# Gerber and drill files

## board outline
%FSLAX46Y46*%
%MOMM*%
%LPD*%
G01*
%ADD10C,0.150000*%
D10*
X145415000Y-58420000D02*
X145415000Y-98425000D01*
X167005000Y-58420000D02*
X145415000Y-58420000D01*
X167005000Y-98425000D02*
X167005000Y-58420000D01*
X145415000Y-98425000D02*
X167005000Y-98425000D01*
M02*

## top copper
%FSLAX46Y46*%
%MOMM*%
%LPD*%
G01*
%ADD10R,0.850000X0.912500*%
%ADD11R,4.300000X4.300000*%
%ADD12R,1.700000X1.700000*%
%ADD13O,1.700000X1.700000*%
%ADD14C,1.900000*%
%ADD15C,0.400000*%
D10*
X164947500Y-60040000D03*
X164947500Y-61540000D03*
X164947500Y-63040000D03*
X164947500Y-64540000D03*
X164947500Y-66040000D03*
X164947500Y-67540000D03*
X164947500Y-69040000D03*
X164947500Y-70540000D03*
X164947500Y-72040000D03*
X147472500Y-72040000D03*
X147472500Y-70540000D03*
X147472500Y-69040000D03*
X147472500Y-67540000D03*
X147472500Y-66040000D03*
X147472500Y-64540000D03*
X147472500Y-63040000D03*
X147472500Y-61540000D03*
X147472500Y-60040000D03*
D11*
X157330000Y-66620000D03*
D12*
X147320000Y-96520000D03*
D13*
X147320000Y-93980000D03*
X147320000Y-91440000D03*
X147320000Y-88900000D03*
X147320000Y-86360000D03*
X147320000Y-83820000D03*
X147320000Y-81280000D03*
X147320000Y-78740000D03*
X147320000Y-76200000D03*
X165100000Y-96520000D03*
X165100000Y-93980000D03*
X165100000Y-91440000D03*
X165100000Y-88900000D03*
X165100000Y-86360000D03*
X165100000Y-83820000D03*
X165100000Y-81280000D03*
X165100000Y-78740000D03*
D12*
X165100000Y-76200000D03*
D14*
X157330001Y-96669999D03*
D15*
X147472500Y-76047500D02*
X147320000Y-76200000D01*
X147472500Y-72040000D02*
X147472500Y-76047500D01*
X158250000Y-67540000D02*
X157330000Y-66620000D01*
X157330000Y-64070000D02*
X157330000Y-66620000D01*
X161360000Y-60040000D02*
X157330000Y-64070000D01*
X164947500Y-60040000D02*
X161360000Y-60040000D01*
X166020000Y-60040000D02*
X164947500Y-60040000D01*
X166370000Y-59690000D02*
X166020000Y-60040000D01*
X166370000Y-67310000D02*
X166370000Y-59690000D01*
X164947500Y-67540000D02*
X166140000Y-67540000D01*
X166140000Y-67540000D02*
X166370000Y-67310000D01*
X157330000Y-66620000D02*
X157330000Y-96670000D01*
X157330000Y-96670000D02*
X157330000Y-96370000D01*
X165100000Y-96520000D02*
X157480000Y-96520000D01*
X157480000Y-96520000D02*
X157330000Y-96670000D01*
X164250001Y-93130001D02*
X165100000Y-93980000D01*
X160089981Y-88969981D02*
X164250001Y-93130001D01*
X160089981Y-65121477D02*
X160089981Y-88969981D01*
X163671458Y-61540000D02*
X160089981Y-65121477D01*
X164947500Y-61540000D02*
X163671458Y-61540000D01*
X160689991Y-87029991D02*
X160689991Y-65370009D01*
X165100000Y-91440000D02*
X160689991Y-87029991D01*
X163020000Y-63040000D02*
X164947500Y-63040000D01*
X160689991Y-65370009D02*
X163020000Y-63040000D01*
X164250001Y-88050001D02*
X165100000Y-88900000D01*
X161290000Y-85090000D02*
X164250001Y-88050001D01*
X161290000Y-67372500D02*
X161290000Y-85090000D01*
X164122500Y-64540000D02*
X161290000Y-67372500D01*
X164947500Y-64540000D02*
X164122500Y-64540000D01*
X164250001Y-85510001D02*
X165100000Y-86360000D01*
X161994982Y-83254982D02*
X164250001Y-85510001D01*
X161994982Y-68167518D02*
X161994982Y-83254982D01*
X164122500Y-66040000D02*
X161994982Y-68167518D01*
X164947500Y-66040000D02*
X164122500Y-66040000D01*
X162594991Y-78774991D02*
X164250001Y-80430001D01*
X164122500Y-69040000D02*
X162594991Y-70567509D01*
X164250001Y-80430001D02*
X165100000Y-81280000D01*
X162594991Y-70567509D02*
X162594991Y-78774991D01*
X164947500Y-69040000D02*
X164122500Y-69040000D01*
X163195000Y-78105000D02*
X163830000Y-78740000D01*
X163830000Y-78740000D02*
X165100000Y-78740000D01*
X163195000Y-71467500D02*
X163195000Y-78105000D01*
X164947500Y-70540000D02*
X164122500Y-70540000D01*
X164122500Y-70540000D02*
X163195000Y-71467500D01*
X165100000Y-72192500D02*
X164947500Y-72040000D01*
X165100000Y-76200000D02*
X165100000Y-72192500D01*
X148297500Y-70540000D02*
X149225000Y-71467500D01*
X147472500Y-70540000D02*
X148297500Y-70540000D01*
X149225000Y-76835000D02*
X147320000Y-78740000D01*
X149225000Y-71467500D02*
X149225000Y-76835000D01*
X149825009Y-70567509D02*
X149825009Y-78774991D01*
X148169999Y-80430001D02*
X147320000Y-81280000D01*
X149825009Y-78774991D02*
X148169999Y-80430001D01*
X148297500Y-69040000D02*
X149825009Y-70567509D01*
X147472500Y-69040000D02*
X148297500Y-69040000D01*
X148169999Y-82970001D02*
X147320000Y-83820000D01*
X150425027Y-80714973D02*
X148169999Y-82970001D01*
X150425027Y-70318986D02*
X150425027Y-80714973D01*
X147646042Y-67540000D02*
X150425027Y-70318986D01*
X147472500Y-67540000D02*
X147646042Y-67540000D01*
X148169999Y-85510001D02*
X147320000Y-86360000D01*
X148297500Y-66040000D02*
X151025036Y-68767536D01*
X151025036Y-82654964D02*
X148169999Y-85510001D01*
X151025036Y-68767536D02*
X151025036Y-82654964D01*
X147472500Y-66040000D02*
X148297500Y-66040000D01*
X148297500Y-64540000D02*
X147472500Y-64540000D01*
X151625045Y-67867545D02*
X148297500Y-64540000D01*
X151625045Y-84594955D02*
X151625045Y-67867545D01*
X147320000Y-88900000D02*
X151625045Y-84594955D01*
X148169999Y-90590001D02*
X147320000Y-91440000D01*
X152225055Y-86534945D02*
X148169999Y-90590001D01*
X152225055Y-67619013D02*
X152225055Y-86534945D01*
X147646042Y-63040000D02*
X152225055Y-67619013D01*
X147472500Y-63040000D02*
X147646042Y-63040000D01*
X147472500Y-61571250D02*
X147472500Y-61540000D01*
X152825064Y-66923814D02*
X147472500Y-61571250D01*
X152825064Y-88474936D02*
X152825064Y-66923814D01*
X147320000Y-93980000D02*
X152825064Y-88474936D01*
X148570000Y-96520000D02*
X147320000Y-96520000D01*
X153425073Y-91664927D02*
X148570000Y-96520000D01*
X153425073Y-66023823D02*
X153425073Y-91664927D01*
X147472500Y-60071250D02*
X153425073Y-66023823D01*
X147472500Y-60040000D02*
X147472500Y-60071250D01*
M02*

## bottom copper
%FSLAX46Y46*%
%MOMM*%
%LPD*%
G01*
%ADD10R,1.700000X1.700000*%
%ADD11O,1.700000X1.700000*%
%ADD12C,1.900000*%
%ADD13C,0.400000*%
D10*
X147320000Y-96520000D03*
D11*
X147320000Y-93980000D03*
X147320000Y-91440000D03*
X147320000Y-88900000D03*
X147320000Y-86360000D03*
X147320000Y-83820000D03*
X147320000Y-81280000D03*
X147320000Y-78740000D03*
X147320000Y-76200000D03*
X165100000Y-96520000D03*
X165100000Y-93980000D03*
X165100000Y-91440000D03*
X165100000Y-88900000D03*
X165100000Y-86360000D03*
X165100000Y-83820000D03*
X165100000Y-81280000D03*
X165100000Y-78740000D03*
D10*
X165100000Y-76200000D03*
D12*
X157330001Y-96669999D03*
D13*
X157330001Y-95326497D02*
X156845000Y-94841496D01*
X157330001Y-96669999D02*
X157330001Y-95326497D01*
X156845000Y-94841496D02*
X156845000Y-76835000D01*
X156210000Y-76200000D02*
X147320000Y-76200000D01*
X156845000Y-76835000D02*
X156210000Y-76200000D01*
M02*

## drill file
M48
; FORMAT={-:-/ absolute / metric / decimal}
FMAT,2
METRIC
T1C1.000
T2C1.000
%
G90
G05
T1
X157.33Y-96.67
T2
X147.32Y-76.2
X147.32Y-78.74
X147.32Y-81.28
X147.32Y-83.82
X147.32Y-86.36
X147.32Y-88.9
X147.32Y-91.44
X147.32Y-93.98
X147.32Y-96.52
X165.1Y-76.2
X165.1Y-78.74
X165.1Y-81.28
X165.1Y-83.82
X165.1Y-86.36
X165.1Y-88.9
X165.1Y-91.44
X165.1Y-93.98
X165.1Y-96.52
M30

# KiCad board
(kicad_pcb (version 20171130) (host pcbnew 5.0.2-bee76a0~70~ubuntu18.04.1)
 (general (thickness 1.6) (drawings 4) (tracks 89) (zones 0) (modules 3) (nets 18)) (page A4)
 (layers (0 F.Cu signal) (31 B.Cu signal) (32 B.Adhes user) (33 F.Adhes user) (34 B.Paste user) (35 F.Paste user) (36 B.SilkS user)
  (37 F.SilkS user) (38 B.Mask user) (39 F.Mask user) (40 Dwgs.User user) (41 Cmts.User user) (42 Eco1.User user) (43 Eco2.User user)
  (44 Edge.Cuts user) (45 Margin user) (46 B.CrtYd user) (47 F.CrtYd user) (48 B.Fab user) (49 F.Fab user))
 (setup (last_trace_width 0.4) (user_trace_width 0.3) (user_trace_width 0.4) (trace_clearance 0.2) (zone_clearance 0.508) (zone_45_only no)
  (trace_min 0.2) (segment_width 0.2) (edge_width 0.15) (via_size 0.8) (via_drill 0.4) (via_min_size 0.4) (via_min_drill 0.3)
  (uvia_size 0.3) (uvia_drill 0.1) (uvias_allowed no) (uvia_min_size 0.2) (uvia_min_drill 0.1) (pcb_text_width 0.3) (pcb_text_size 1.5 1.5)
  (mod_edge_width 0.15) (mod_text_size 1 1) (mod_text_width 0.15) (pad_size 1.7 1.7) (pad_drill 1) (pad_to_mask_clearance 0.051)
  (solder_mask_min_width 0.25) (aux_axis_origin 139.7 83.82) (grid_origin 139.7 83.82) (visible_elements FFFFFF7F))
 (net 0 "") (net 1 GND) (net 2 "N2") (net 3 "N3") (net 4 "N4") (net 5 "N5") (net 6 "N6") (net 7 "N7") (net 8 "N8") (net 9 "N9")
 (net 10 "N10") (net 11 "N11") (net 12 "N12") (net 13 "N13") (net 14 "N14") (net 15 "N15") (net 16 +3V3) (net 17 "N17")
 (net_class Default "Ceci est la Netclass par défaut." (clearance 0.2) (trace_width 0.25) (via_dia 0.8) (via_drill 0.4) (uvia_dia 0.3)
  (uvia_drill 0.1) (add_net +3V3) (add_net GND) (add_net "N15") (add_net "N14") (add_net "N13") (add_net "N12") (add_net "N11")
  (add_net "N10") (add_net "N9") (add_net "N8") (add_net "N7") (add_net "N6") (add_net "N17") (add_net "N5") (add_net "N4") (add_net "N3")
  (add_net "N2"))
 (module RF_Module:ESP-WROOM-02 (layer F.Cu) (at 156.21 66.04)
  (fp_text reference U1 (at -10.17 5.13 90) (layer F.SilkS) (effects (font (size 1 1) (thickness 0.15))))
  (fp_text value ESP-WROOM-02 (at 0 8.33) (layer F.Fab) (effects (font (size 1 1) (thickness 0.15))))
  (pad 18 smd rect (at 8.7375 -6) (size 0.85 0.9125) (layers F.Cu F.Paste F.Mask) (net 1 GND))
  (pad 17 smd rect (at 8.7375 -4.5) (size 0.85 0.9125) (layers F.Cu F.Paste F.Mask) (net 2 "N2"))
  (pad 16 smd rect (at 8.7375 -3) (size 0.85 0.9125) (layers F.Cu F.Paste F.Mask) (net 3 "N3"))
  (pad 15 smd rect (at 8.7375 -1.5) (size 0.85 0.9125) (layers F.Cu F.Paste F.Mask) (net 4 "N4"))
  (pad 14 smd rect (at 8.7375 0) (size 0.85 0.9125) (layers F.Cu F.Paste F.Mask) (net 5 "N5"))
  (pad 13 smd rect (at 8.7375 1.5) (size 0.85 0.9125) (layers F.Cu F.Paste F.Mask) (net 1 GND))
  (pad 12 smd rect (at 8.7375 3) (size 0.85 0.9125) (layers F.Cu F.Paste F.Mask) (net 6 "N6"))
  (pad 11 smd rect (at 8.7375 4.5) (size 0.85 0.9125) (layers F.Cu F.Paste F.Mask) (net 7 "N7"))
  (pad 10 smd rect (at 8.7375 6) (size 0.85 0.9125) (layers F.Cu F.Paste F.Mask) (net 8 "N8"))
  (pad 9 smd rect (at -8.7375 6) (size 0.85 0.9125) (layers F.Cu F.Paste F.Mask) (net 1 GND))
  (pad 8 smd rect (at -8.7375 4.5) (size 0.85 0.9125) (layers F.Cu F.Paste F.Mask) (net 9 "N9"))
  (pad 7 smd rect (at -8.7375 3) (size 0.85 0.9125) (layers F.Cu F.Paste F.Mask) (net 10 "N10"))
  (pad 6 smd rect (at -8.7375 1.5) (size 0.85 0.9125) (layers F.Cu F.Paste F.Mask) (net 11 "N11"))
  (pad 5 smd rect (at -8.7375 0) (size 0.85 0.9125) (layers F.Cu F.Paste F.Mask) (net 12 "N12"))
  (pad 4 smd rect (at -8.7375 -1.5) (size 0.85 0.9125) (layers F.Cu F.Paste F.Mask) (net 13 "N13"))
  (pad 3 smd rect (at -8.7375 -3) (size 0.85 0.9125) (layers F.Cu F.Paste F.Mask) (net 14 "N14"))
  (pad 2 smd rect (at -8.7375 -4.5) (size 0.85 0.9125) (layers F.Cu F.Paste F.Mask) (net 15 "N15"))
  (pad 1 smd rect (at -8.7375 -6) (size 0.85 0.9125) (layers F.Cu F.Paste F.Mask) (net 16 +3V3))
  (pad 19 smd rect (at 1.12 0.58) (size 4.3 4.3) (layers F.Cu F.Paste F.Mask) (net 1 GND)))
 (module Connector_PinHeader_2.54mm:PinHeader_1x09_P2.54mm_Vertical (layer F.Cu) (at 147.32 96.52 180)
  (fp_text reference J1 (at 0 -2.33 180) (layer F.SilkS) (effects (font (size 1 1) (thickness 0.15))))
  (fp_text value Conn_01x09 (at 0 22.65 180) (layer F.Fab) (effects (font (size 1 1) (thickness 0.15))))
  (pad 1 thru_hole rect (at 0 0 180) (size 1.7 1.7) (drill 1) (layers *.Cu *.Mask) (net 16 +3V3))
  (pad 2 thru_hole oval (at 0 2.54 180) (size 1.7 1.7) (drill 1) (layers *.Cu *.Mask) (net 15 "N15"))
  (pad 3 thru_hole oval (at 0 5.08 180) (size 1.7 1.7) (drill 1) (layers *.Cu *.Mask) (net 14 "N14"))
  (pad 4 thru_hole oval (at 0 7.62 180) (size 1.7 1.7) (drill 1) (layers *.Cu *.Mask) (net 13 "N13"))
  (pad 5 thru_hole oval (at 0 10.16 180) (size 1.7 1.7) (drill 1) (layers *.Cu *.Mask) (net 12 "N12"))
  (pad 6 thru_hole oval (at 0 12.7 180) (size 1.7 1.7) (drill 1) (layers *.Cu *.Mask) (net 11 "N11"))
  (pad 7 thru_hole oval (at 0 15.24 180) (size 1.7 1.7) (drill 1) (layers *.Cu *.Mask) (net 10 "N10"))
  (pad 8 thru_hole oval (at 0 17.78 180) (size 1.7 1.7) (drill 1) (layers *.Cu *.Mask) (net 9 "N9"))
  (pad 9 thru_hole oval (at 0 20.32 180) (size 1.7 1.7) (drill 1) (layers *.Cu *.Mask) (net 1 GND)))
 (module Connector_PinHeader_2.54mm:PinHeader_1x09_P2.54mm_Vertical (layer F.Cu) (at 165.1 76.2)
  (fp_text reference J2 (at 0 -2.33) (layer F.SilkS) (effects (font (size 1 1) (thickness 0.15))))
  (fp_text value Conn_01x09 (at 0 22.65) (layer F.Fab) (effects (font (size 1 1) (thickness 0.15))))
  (pad 9 thru_hole oval (at 0 20.32) (size 1.7 1.7) (drill 1) (layers *.Cu *.Mask) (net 1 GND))
  (pad 8 thru_hole oval (at 0 17.78) (size 1.7 1.7) (drill 1) (layers *.Cu *.Mask) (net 2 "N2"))
  (pad 7 thru_hole oval (at 0 15.24) (size 1.7 1.7) (drill 1) (layers *.Cu *.Mask) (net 3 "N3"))
  (pad 6 thru_hole oval (at 0 12.7) (size 1.7 1.7) (drill 1) (layers *.Cu *.Mask) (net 4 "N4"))
  (pad 5 thru_hole oval (at 0 10.16) (size 1.7 1.7) (drill 1) (layers *.Cu *.Mask) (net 5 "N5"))
  (pad 4 thru_hole oval (at 0 7.62) (size 1.7 1.7) (drill 1) (layers *.Cu *.Mask) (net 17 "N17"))
  (pad 3 thru_hole oval (at 0 5.08) (size 1.7 1.7) (drill 1) (layers *.Cu *.Mask) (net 6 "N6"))
  (pad 2 thru_hole oval (at 0 2.54) (size 1.7 1.7) (drill 1) (layers *.Cu *.Mask) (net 7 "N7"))
  (pad 1 thru_hole rect (at 0 0) (size 1.7 1.7) (drill 1) (layers *.Cu *.Mask) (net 8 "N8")))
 (gr_line (start 145.415 58.42) (end 145.415 98.425) (layer Edge.Cuts) (width 0.15))
 (gr_line (start 167.005 58.42) (end 145.415 58.42) (layer Edge.Cuts) (width 0.15))
 (gr_line (start 167.005 98.425) (end 167.005 58.42) (layer Edge.Cuts) (width 0.15))
 (gr_line (start 145.415 98.425) (end 167.005 98.425) (layer Edge.Cuts) (width 0.15))
 (segment (start 147.4725 76.0475) (end 147.32 76.2) (width 0.4) (layer F.Cu) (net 1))
 (segment (start 147.4725 72.04) (end 147.4725 76.0475) (width 0.4) (layer F.Cu) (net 1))
 (segment (start 158.25 67.54) (end 157.33 66.62) (width 0.4) (layer F.Cu) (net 1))
 (segment (start 157.33 64.07) (end 157.33 66.62) (width 0.4) (layer F.Cu) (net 1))
 (segment (start 161.36 60.04) (end 157.33 64.07) (width 0.4) (layer F.Cu) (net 1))
 (segment (start 164.9475 60.04) (end 161.36 60.04) (width 0.4) (layer F.Cu) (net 1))
 (segment (start 166.02 60.04) (end 164.9475 60.04) (width 0.4) (layer F.Cu) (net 1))
 (segment (start 166.37 59.69) (end 166.02 60.04) (width 0.4) (layer F.Cu) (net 1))
 (segment (start 166.37 67.31) (end 166.37 59.69) (width 0.4) (layer F.Cu) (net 1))
 (segment (start 164.9475 67.54) (end 166.14 67.54) (width 0.4) (layer F.Cu) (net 1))
 (segment (start 166.14 67.54) (end 166.37 67.31) (width 0.4) (layer F.Cu) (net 1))
 (segment (start 157.33 66.62) (end 157.33 96.67) (width 0.4) (layer F.Cu) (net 1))
 (segment (start 157.33 96.67) (end 157.33 96.37) (width 0.4) (layer F.Cu) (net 1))
 (segment (start 165.1 96.52) (end 157.48 96.52) (width 0.4) (layer F.Cu) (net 1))
 (segment (start 157.48 96.52) (end 157.33 96.67) (width 0.4) (layer F.Cu) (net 1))
 (via (at 157.330001 96.669999) (size 1.9) (drill 1) (layers F.Cu B.Cu) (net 1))
 (segment (start 157.330001 95.326497) (end 156.845 94.841496) (width 0.4) (layer B.Cu) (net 1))
 (segment (start 157.330001 96.669999) (end 157.330001 95.326497) (width 0.4) (layer B.Cu) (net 1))
 (segment (start 156.845 94.841496) (end 156.845 76.835) (width 0.4) (layer B.Cu) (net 1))
 (segment (start 156.21 76.2) (end 147.32 76.2) (width 0.4) (layer B.Cu) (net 1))
 (segment (start 156.845 76.835) (end 156.21 76.2) (width 0.4) (layer B.Cu) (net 1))
 (segment (start 164.250001 93.130001) (end 165.1 93.98) (width 0.4) (layer F.Cu) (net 2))
 (segment (start 160.089981 88.969981) (end 164.250001 93.130001) (width 0.4) (layer F.Cu) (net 2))
 (segment (start 160.089981 65.121477) (end 160.089981 88.969981) (width 0.4) (layer F.Cu) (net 2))
 (segment (start 163.671458 61.54) (end 160.089981 65.121477) (width 0.4) (layer F.Cu) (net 2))
 (segment (start 164.9475 61.54) (end 163.671458 61.54) (width 0.4) (layer F.Cu) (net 2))
 (segment (start 160.689991 87.029991) (end 160.689991 65.370009) (width 0.4) (layer F.Cu) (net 3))
 (segment (start 165.1 91.44) (end 160.689991 87.029991) (width 0.4) (layer F.Cu) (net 3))
 (segment (start 163.02 63.04) (end 164.9475 63.04) (width 0.4) (layer F.Cu) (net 3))
 (segment (start 160.689991 65.370009) (end 163.02 63.04) (width 0.4) (layer F.Cu) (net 3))
 (segment (start 164.250001 88.050001) (end 165.1 88.9) (width 0.4) (layer F.Cu) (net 4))
 (segment (start 161.29 85.09) (end 164.250001 88.050001) (width 0.4) (layer F.Cu) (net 4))
 (segment (start 161.29 67.3725) (end 161.29 85.09) (width 0.4) (layer F.Cu) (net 4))
 (segment (start 164.1225 64.54) (end 161.29 67.3725) (width 0.4) (layer F.Cu) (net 4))
 (segment (start 164.9475 64.54) (end 164.1225 64.54) (width 0.4) (layer F.Cu) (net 4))
 (segment (start 164.250001 85.510001) (end 165.1 86.36) (width 0.4) (layer F.Cu) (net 5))
 (segment (start 161.994982 83.254982) (end 164.250001 85.510001) (width 0.4) (layer F.Cu) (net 5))
 (segment (start 161.994982 68.167518) (end 161.994982 83.254982) (width 0.4) (layer F.Cu) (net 5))
 (segment (start 164.1225 66.04) (end 161.994982 68.167518) (width 0.4) (layer F.Cu) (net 5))
 (segment (start 164.9475 66.04) (end 164.1225 66.04) (width 0.4) (layer F.Cu) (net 5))
 (segment (start 162.594991 78.774991) (end 164.250001 80.430001) (width 0.4) (layer F.Cu) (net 6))
 (segment (start 164.1225 69.04) (end 162.594991 70.567509) (width 0.4) (layer F.Cu) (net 6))
 (segment (start 164.250001 80.430001) (end 165.1 81.28) (width 0.4) (layer F.Cu) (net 6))
 (segment (start 162.594991 70.567509) (end 162.594991 78.774991) (width 0.4) (layer F.Cu) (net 6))
 (segment (start 164.9475 69.04) (end 164.1225 69.04) (width 0.4) (layer F.Cu) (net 6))
 (segment (start 163.195 78.105) (end 163.83 78.74) (width 0.4) (layer F.Cu) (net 7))
 (segment (start 163.83 78.74) (end 165.1 78.74) (width 0.4) (layer F.Cu) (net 7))
 (segment (start 163.195 71.4675) (end 163.195 78.105) (width 0.4) (layer F.Cu) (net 7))
 (segment (start 164.9475 70.54) (end 164.1225 70.54) (width 0.4) (layer F.Cu) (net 7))
 (segment (start 164.1225 70.54) (end 163.195 71.4675) (width 0.4) (layer F.Cu) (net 7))
 (segment (start 165.1 72.1925) (end 164.9475 72.04) (width 0.4) (layer F.Cu) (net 8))
 (segment (start 165.1 76.2) (end 165.1 72.1925) (width 0.4) (layer F.Cu) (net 8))
 (segment (start 148.2975 70.54) (end 149.225 71.4675) (width 0.4) (layer F.Cu) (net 9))
 (segment (start 147.4725 70.54) (end 148.2975 70.54) (width 0.4) (layer F.Cu) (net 9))
 (segment (start 149.225 76.835) (end 147.32 78.74) (width 0.4) (layer F.Cu) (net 9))
 (segment (start 149.225 71.4675) (end 149.225 76.835) (width 0.4) (layer F.Cu) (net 9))
 (segment (start 149.825009 70.567509) (end 149.825009 78.774991) (width 0.4) (layer F.Cu) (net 10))
 (segment (start 148.169999 80.430001) (end 147.32 81.28) (width 0.4) (layer F.Cu) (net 10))
 (segment (start 149.825009 78.774991) (end 148.169999 80.430001) (width 0.4) (layer F.Cu) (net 10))
 (segment (start 148.2975 69.04) (end 149.825009 70.567509) (width 0.4) (layer F.Cu) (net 10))
 (segment (start 147.4725 69.04) (end 148.2975 69.04) (width 0.4) (layer F.Cu) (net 10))
 (segment (start 148.169999 82.970001) (end 147.32 83.82) (width 0.4) (layer F.Cu) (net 11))
 (segment (start 150.425027 80.714973) (end 148.169999 82.970001) (width 0.4) (layer F.Cu) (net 11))
 (segment (start 150.425027 70.318986) (end 150.425027 80.714973) (width 0.4) (layer F.Cu) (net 11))
 (segment (start 147.646042 67.54) (end 150.425027 70.318986) (width 0.4) (layer F.Cu) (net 11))
 (segment (start 147.4725 67.54) (end 147.646042 67.54) (width 0.4) (layer F.Cu) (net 11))
 (segment (start 148.169999 85.510001) (end 147.32 86.36) (width 0.4) (layer F.Cu) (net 12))
 (segment (start 148.2975 66.04) (end 151.025036 68.767536) (width 0.4) (layer F.Cu) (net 12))
 (segment (start 151.025036 82.654964) (end 148.169999 85.510001) (width 0.4) (layer F.Cu) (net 12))
 (segment (start 151.025036 68.767536) (end 151.025036 82.654964) (width 0.4) (layer F.Cu) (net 12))
 (segment (start 147.4725 66.04) (end 148.2975 66.04) (width 0.4) (layer F.Cu) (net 12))
 (segment (start 148.2975 64.54) (end 147.4725 64.54) (width 0.4) (layer F.Cu) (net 13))
 (segment (start 151.625045 67.867545) (end 148.2975 64.54) (width 0.4) (layer F.Cu) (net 13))
 (segment (start 151.625045 84.594955) (end 151.625045 67.867545) (width 0.4) (layer F.Cu) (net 13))
 (segment (start 147.32 88.9) (end 151.625045 84.594955) (width 0.4) (layer F.Cu) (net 13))
 (segment (start 148.169999 90.590001) (end 147.32 91.44) (width 0.4) (layer F.Cu) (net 14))
 (segment (start 152.225055 86.534945) (end 148.169999 90.590001) (width 0.4) (layer F.Cu) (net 14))
 (segment (start 152.225055 67.619013) (end 152.225055 86.534945) (width 0.4) (layer F.Cu) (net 14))
 (segment (start 147.646042 63.04) (end 152.225055 67.619013) (width 0.4) (layer F.Cu) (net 14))
 (segment (start 147.4725 63.04) (end 147.646042 63.04) (width 0.4) (layer F.Cu) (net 14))
 (segment (start 147.4725 61.57125) (end 147.4725 61.54) (width 0.4) (layer F.Cu) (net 15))
 (segment (start 152.825064 66.923814) (end 147.4725 61.57125) (width 0.4) (layer F.Cu) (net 15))
 (segment (start 152.825064 88.474936) (end 152.825064 66.923814) (width 0.4) (layer F.Cu) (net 15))
 (segment (start 147.32 93.98) (end 152.825064 88.474936) (width 0.4) (layer F.Cu) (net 15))
 (segment (start 148.57 96.52) (end 147.32 96.52) (width 0.4) (layer F.Cu) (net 16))
 (segment (start 153.425073 91.664927) (end 148.57 96.52) (width 0.4) (layer F.Cu) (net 16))
 (segment (start 153.425073 66.023823) (end 153.425073 91.664927) (width 0.4) (layer F.Cu) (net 16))
 (segment (start 147.4725 60.07125) (end 153.425073 66.023823) (width 0.4) (layer F.Cu) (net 16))
 (segment (start 147.4725 60.04) (end 147.4725 60.07125) (width 0.4) (layer F.Cu) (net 16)))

